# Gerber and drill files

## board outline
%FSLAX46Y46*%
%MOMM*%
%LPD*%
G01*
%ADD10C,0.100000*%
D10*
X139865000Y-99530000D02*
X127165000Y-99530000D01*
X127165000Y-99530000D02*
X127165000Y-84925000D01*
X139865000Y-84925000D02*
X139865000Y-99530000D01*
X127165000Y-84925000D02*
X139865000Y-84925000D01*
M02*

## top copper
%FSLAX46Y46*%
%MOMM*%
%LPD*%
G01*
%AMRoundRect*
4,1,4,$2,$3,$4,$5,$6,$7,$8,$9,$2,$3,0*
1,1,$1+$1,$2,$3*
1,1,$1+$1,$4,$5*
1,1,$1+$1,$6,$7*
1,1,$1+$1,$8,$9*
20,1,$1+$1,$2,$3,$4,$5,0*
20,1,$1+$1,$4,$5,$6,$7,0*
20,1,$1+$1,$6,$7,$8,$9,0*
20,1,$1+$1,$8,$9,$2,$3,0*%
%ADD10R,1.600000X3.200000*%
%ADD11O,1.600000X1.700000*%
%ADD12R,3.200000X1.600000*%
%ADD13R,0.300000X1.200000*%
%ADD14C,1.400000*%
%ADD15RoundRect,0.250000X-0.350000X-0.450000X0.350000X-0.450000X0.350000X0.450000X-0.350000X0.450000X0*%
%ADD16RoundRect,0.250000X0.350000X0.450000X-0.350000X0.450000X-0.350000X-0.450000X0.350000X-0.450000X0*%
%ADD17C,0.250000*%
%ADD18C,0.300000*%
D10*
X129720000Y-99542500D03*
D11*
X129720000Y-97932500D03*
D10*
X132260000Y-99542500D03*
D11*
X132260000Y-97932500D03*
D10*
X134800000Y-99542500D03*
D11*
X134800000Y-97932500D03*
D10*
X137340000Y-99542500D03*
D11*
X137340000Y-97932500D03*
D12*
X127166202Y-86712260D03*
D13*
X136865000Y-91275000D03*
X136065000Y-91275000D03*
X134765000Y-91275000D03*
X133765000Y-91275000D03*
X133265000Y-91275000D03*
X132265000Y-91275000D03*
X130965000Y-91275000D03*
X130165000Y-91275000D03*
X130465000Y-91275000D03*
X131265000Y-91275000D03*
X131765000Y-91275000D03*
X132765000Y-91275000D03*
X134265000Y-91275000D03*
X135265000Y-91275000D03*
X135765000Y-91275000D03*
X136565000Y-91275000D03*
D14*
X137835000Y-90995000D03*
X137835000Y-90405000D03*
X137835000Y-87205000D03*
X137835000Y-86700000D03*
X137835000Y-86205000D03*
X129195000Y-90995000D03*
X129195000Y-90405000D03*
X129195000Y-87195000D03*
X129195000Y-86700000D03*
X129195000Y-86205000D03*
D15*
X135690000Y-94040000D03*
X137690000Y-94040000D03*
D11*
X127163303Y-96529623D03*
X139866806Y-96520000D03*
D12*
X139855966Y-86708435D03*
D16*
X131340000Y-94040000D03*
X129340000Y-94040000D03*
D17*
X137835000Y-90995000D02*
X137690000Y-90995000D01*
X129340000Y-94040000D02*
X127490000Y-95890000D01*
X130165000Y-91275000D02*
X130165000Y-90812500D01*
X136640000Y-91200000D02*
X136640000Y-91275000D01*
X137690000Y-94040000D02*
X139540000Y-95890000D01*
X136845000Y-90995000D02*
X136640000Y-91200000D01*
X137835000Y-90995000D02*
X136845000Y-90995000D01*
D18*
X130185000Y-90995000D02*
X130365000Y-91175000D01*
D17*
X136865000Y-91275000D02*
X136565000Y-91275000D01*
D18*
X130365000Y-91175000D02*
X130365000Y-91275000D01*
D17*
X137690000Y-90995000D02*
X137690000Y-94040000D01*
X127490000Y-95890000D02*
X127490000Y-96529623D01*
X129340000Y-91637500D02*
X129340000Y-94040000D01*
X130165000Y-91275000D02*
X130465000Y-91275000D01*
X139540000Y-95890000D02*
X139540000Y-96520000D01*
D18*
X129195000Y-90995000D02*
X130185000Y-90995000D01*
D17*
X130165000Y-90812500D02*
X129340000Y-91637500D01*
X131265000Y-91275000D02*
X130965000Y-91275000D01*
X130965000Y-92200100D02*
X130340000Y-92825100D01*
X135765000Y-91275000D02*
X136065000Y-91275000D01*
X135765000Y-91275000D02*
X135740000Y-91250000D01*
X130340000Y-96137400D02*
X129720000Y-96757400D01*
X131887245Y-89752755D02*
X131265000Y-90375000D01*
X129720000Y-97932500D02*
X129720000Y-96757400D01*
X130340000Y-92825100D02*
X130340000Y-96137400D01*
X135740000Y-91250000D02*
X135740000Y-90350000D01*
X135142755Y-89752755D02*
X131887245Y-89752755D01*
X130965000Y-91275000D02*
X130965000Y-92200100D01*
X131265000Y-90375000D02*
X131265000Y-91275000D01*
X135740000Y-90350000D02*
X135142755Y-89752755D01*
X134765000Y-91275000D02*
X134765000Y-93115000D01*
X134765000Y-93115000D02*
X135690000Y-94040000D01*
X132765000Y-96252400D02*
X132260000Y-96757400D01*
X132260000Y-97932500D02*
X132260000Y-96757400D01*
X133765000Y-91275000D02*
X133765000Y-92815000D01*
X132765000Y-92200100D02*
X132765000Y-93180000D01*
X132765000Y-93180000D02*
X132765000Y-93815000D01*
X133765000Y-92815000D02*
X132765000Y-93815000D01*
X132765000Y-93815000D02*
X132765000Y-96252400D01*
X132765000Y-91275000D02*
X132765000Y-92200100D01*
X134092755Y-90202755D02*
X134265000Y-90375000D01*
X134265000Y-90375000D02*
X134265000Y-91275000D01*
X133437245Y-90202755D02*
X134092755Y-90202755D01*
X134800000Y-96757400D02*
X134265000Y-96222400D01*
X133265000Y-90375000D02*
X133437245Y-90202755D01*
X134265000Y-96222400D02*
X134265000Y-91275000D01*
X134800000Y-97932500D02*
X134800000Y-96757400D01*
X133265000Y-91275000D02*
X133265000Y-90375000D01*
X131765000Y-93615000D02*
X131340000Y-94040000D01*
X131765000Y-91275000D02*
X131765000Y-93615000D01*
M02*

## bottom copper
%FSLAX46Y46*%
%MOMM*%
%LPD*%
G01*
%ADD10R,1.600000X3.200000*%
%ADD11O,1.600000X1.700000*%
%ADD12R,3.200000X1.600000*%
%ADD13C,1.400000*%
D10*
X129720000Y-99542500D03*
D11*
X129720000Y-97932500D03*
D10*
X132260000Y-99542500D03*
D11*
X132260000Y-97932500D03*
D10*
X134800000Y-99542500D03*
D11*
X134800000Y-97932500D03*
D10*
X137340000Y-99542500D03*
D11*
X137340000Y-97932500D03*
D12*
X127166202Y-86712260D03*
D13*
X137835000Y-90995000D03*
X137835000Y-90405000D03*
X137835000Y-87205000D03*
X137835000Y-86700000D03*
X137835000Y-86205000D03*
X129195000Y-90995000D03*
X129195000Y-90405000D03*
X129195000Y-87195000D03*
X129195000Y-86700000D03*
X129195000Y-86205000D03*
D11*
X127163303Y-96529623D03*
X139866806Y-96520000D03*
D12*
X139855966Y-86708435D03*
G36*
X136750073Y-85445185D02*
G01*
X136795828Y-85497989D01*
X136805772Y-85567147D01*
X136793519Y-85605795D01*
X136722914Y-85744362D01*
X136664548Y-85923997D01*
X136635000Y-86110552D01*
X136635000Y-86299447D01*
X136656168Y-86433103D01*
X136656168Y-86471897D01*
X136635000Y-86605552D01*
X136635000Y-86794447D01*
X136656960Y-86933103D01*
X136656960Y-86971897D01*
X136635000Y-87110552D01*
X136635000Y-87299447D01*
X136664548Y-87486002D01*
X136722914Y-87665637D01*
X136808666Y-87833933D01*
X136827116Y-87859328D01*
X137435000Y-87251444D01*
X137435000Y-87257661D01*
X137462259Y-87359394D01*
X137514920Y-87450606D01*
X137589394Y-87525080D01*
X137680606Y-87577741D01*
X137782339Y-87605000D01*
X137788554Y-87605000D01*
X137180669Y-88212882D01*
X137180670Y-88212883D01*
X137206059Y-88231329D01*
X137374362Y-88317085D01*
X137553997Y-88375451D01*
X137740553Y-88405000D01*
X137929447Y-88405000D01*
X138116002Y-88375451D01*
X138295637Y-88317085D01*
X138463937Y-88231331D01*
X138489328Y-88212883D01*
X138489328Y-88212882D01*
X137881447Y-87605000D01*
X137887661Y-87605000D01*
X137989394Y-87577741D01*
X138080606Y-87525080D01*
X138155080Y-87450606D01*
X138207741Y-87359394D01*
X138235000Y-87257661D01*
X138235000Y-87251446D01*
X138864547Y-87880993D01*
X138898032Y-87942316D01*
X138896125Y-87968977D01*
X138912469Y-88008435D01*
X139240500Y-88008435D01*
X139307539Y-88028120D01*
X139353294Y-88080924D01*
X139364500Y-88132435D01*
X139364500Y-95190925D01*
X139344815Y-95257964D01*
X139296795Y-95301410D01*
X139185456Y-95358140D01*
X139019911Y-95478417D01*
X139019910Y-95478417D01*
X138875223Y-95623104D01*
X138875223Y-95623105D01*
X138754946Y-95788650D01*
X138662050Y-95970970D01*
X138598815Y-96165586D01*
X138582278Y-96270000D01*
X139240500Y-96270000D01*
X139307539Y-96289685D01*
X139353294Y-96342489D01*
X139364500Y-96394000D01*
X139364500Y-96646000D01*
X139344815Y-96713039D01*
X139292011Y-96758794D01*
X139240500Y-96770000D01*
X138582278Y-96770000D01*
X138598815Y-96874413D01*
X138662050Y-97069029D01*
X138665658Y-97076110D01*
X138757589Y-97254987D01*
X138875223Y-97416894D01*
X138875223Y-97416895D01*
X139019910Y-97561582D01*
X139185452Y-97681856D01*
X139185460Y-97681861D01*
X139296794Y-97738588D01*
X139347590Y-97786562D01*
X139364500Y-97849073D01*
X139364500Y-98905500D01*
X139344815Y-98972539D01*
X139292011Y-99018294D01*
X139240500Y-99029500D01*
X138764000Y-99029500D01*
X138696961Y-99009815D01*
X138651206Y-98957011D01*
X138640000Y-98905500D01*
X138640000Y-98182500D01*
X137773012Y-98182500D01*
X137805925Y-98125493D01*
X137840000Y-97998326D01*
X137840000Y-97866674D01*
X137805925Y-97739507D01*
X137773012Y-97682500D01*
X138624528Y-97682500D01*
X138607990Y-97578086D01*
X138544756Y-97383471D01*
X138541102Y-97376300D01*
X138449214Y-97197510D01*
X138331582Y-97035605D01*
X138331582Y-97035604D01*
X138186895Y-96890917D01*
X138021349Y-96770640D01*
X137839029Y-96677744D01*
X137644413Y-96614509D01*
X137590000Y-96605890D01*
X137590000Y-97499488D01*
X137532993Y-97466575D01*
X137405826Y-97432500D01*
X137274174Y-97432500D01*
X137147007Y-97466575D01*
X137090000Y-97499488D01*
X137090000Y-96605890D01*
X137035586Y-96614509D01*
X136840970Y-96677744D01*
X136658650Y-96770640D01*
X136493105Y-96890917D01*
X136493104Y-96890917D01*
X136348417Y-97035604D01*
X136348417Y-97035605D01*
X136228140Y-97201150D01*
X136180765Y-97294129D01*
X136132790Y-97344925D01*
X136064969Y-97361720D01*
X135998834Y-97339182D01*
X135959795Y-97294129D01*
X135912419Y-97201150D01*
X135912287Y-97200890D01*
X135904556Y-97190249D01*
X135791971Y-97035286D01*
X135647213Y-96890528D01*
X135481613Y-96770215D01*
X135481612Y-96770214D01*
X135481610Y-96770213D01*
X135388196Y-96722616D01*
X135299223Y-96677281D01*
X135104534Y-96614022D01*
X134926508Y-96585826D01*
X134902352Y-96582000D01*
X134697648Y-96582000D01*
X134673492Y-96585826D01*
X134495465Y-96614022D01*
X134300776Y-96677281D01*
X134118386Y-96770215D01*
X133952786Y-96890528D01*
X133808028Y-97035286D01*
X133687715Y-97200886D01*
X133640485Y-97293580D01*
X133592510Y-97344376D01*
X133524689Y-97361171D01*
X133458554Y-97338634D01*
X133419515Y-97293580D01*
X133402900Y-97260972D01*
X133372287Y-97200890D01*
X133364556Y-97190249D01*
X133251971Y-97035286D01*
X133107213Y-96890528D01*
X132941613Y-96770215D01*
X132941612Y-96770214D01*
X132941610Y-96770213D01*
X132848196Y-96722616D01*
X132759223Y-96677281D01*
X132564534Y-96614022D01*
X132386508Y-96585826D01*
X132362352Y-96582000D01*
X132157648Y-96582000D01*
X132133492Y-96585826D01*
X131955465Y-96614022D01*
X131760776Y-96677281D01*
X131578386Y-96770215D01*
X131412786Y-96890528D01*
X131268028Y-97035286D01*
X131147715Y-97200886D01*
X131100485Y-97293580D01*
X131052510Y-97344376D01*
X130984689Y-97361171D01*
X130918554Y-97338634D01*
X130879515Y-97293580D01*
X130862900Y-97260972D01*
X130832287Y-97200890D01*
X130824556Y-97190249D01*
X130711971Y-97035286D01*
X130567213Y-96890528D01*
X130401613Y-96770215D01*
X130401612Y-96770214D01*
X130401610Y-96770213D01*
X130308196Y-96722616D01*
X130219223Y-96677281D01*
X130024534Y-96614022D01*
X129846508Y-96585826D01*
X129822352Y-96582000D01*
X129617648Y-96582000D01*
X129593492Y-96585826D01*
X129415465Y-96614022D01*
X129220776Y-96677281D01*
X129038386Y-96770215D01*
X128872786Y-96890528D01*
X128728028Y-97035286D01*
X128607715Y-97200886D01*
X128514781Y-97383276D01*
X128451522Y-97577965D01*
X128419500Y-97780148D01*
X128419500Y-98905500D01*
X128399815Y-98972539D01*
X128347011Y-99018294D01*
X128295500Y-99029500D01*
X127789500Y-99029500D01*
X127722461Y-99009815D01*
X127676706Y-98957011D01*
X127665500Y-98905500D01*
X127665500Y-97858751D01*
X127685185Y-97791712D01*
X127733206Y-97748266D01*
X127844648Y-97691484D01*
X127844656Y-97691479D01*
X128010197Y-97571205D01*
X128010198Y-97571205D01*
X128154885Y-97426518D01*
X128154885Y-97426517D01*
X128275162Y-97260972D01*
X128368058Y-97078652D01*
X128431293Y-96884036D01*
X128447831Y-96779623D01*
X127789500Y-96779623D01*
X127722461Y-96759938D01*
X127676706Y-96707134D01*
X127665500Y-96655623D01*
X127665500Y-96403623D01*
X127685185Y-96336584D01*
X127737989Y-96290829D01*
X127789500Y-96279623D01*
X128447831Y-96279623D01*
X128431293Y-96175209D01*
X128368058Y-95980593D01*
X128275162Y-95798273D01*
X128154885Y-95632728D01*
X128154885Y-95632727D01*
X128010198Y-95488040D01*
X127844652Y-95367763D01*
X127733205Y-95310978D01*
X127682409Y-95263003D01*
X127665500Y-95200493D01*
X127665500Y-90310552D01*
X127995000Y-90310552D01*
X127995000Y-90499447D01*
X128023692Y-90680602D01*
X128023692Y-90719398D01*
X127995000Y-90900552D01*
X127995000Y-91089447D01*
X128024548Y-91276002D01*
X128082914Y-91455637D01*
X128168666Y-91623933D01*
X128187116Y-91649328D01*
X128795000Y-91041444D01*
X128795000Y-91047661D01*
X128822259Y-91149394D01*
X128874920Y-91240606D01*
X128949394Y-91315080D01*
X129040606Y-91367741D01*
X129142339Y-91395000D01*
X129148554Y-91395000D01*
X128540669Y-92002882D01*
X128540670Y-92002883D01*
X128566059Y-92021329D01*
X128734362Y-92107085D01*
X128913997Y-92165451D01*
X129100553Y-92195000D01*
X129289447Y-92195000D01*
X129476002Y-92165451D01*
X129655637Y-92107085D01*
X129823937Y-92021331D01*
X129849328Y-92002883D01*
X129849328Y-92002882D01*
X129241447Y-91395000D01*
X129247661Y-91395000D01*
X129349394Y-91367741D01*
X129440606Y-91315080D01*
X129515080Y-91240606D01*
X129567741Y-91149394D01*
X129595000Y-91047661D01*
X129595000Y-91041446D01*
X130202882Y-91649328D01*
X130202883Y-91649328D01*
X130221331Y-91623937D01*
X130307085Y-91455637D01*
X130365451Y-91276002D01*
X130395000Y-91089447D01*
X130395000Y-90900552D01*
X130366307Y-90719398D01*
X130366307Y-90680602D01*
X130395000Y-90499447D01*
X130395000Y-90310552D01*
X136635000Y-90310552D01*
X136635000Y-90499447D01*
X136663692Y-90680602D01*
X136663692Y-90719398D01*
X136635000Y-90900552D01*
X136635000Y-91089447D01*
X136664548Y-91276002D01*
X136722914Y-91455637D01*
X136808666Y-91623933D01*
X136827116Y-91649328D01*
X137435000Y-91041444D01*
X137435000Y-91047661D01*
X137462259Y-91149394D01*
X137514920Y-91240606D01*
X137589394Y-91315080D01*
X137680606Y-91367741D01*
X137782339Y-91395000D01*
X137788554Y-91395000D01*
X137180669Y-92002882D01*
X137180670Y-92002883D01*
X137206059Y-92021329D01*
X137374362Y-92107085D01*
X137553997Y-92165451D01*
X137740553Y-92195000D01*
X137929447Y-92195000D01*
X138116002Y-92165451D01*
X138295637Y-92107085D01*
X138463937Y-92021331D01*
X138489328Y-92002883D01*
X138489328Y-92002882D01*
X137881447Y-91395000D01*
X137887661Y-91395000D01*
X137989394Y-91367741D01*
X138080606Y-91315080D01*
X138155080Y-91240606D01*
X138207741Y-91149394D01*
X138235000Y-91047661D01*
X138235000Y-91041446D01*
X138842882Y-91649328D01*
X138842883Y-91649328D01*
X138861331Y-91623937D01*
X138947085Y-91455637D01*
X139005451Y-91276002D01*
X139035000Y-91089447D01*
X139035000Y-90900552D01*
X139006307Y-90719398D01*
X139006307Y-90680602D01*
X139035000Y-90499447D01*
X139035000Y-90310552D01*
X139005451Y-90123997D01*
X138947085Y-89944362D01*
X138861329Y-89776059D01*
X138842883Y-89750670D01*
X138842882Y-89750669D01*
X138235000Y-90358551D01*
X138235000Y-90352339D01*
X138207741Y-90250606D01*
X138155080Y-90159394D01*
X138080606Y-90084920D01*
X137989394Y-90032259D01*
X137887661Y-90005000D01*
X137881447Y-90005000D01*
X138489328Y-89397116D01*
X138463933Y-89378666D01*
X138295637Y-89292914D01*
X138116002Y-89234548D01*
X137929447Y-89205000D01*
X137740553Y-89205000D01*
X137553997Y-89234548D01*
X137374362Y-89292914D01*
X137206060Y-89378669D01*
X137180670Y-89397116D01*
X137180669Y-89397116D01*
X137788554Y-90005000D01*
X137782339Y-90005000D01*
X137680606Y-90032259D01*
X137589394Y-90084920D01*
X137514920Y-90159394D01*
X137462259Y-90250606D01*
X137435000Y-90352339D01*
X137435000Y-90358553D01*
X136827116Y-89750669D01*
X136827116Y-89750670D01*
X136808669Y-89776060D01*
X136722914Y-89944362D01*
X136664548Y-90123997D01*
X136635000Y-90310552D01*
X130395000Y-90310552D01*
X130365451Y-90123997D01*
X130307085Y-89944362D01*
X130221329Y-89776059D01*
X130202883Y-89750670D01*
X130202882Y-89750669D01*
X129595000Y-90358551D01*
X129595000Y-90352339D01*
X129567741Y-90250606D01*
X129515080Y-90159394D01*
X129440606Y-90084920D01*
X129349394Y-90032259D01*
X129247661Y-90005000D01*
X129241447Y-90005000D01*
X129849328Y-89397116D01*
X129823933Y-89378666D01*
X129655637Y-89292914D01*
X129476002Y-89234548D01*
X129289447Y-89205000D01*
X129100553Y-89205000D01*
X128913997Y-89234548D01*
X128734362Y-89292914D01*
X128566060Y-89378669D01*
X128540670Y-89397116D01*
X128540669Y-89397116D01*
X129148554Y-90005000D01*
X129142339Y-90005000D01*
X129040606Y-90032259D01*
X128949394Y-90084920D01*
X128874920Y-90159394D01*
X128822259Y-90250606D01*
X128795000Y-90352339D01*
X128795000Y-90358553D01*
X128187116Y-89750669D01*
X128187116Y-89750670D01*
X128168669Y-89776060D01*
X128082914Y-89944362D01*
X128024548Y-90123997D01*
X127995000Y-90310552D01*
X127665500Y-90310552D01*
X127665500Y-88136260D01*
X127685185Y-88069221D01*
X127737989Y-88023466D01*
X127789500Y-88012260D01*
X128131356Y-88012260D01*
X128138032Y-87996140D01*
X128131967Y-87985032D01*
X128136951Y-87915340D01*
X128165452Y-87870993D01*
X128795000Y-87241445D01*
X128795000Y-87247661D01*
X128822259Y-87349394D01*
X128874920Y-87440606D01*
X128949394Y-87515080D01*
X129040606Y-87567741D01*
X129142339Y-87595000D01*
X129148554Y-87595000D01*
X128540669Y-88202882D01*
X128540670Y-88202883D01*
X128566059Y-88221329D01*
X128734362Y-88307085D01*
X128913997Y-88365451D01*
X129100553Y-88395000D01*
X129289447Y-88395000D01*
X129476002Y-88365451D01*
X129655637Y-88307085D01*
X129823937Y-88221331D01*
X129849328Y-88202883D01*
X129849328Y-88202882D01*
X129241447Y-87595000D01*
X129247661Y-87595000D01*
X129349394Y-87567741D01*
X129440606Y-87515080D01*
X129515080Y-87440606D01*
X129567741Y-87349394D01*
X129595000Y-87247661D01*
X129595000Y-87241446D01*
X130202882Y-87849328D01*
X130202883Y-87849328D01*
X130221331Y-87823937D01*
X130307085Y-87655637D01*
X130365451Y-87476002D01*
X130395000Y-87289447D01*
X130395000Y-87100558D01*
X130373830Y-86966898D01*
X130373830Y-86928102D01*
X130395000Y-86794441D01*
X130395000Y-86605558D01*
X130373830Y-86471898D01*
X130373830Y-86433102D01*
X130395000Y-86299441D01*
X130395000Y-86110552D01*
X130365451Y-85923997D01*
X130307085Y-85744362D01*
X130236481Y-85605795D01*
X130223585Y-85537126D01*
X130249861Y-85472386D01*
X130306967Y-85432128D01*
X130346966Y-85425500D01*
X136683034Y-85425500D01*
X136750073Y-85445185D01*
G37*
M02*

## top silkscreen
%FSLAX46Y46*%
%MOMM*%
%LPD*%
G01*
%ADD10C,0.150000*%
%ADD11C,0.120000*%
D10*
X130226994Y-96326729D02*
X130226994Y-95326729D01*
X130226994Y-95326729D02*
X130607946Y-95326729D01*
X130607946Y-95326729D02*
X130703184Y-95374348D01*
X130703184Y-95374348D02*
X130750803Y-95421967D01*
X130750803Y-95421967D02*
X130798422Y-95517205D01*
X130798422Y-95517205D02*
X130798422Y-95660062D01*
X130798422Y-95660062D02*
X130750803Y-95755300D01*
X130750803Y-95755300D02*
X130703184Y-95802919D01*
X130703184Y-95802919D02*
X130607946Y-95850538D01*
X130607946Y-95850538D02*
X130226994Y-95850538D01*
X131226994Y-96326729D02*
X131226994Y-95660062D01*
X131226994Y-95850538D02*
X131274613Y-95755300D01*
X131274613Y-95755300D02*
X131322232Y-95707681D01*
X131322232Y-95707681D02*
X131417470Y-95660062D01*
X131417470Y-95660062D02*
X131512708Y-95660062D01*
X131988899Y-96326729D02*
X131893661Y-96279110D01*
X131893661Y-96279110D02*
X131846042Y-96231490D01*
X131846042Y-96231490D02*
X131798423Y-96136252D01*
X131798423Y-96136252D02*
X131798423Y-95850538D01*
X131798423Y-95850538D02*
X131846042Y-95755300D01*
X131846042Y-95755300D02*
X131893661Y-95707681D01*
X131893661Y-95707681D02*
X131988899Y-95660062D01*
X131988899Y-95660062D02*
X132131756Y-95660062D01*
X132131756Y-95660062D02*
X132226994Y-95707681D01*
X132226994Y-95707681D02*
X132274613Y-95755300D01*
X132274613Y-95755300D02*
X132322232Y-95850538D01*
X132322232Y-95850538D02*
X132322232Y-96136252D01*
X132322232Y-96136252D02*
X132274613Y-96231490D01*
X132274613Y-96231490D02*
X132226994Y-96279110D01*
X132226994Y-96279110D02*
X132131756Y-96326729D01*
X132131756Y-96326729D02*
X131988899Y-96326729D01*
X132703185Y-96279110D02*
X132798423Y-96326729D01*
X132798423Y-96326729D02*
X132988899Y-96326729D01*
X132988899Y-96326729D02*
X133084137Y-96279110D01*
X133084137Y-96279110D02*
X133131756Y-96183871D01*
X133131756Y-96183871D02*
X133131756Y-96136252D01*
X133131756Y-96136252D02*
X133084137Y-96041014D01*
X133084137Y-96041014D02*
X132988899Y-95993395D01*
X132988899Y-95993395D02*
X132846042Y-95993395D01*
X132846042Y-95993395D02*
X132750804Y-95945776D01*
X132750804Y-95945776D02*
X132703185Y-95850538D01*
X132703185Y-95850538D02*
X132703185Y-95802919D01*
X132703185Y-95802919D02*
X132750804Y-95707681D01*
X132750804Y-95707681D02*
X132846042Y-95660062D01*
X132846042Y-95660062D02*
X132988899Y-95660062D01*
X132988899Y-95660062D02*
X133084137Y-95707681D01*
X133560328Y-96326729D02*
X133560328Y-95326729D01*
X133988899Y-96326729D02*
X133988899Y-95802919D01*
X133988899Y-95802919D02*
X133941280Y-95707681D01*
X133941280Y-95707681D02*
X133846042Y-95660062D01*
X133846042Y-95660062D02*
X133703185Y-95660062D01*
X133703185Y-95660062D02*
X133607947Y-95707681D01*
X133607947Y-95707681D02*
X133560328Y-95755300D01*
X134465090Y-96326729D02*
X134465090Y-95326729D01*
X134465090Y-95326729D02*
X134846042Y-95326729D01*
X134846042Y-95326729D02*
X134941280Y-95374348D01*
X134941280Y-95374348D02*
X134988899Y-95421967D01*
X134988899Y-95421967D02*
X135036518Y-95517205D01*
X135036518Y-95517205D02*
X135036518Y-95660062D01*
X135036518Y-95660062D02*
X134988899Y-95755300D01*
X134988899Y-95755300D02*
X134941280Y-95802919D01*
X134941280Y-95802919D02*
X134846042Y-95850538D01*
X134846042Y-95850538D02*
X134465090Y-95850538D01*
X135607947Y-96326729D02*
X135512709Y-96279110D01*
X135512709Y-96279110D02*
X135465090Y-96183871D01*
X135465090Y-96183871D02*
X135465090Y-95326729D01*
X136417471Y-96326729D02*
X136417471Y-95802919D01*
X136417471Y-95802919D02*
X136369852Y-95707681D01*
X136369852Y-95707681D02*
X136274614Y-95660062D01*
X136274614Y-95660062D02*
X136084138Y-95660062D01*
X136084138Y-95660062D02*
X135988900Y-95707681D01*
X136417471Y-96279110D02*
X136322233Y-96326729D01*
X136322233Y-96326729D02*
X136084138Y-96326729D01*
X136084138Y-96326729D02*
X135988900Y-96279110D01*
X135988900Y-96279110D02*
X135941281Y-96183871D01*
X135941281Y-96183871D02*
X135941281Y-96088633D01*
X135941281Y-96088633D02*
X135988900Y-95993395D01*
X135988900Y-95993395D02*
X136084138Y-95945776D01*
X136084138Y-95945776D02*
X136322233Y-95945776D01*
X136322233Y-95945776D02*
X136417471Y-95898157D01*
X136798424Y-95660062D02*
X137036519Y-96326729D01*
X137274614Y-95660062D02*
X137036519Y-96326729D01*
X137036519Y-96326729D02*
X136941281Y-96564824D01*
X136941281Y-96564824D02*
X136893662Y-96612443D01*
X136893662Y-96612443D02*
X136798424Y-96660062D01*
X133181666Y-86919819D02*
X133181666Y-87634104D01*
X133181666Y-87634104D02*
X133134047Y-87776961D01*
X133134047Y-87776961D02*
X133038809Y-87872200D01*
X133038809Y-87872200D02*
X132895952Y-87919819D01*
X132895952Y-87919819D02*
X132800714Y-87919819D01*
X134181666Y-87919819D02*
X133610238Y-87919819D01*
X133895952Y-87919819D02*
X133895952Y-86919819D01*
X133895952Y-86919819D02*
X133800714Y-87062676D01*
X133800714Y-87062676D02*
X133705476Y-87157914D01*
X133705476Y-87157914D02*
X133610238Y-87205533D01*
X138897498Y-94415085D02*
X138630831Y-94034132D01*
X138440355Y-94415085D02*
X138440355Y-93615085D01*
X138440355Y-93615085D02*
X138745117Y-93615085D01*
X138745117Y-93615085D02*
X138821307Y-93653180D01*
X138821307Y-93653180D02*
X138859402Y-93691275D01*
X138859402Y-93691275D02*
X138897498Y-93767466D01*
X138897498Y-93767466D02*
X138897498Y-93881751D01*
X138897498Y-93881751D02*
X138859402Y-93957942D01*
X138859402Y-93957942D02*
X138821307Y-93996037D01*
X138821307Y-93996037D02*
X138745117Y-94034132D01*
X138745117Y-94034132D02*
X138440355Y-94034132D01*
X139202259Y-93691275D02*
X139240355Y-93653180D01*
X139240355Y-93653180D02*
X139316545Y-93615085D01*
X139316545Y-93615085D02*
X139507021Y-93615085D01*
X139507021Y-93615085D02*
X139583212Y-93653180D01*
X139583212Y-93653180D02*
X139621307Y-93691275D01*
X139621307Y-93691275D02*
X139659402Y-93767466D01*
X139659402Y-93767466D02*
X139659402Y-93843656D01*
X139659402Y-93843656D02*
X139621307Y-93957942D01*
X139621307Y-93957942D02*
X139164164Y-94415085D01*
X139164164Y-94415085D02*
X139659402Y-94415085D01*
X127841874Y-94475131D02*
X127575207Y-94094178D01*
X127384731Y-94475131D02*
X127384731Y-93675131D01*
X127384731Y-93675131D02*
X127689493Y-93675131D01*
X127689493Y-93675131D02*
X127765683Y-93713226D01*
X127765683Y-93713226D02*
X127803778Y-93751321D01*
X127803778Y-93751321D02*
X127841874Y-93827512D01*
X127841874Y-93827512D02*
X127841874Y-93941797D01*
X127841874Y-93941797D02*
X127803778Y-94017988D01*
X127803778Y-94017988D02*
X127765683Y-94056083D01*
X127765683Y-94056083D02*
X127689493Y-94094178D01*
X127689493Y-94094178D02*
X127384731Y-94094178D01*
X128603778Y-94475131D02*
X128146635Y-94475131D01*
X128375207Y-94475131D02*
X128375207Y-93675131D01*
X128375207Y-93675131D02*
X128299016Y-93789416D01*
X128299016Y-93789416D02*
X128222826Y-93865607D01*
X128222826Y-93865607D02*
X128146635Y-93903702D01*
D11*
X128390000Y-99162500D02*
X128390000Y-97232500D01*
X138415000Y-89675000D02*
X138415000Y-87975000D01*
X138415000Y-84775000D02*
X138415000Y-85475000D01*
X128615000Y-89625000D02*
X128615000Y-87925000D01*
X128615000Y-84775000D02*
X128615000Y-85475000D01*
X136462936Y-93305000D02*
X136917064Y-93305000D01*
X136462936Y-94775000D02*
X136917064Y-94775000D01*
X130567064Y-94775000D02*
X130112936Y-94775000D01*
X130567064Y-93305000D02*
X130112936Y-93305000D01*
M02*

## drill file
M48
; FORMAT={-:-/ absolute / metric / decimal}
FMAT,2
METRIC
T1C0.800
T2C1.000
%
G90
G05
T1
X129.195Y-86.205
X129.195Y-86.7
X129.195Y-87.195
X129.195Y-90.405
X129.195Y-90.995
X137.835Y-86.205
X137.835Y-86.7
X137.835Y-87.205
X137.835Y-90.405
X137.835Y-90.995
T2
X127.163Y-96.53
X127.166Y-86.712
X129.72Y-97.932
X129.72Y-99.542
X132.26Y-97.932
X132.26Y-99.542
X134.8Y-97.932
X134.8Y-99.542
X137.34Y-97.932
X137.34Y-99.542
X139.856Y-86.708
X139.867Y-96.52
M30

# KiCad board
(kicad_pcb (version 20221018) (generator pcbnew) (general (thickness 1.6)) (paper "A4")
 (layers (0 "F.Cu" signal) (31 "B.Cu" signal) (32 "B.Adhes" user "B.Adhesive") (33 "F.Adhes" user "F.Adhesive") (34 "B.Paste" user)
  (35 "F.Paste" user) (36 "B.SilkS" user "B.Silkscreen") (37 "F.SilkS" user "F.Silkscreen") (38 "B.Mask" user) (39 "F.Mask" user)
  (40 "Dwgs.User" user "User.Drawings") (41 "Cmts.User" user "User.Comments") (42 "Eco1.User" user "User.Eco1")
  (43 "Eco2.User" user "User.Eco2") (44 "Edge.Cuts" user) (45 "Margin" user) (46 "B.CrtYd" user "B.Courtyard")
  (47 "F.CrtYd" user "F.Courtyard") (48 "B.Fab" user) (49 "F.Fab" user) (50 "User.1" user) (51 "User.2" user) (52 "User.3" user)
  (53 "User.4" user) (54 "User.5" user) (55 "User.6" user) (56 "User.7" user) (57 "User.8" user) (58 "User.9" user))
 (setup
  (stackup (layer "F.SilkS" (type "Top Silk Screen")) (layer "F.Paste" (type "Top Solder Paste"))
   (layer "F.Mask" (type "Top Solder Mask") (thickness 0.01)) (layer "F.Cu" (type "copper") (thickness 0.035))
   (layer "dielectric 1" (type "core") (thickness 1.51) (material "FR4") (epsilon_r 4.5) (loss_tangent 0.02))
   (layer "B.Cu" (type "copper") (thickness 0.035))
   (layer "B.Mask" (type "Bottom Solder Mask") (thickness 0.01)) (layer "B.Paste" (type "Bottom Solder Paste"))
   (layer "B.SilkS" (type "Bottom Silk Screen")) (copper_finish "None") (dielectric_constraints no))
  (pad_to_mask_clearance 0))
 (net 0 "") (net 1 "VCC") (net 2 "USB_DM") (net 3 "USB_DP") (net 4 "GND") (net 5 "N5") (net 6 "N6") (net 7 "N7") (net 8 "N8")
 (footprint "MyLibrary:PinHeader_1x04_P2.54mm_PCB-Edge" (layer "F.Cu") (at 129.72 97.9325 90)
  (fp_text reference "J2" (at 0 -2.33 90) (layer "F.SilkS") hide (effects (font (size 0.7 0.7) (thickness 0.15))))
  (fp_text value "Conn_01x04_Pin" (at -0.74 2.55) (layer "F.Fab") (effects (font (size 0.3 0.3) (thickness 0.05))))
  (fp_line (start -1.23 -1.33) (end 0.7 -1.33) (stroke (width 0.12) (type solid)) (layer "F.SilkS"))
  (pad "1" thru_hole rect (at -1.61 0 90) (size 3.2 1.6) (drill 1) (layers "*.Cu" "*.Mask") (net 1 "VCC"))
  (pad "1" thru_hole oval (at 0 0 90) (size 1.7 1.6) (drill 1) (layers "*.Cu" "*.Mask") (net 1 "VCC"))
  (pad "2" thru_hole rect (at -1.61 2.54 90) (size 3.2 1.6) (drill 1) (layers "*.Cu" "*.Mask") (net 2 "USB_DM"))
  (pad "2" thru_hole oval (at 0 2.54 90) (size 1.7 1.6) (drill 1) (layers "*.Cu" "*.Mask") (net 2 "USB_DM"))
  (pad "3" thru_hole rect (at -1.61 5.08 90) (size 3.2 1.6) (drill 1) (layers "*.Cu" "*.Mask") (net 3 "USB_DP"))
  (pad "3" thru_hole oval (at 0 5.08 90) (size 1.7 1.6) (drill 1) (layers "*.Cu" "*.Mask") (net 3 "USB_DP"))
  (pad "4" thru_hole rect (at -1.61 7.62 90) (size 3.2 1.6) (drill 1) (layers "*.Cu" "*.Mask") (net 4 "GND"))
  (pad "4" thru_hole oval (at 0 7.62 90) (size 1.7 1.6) (drill 1) (layers "*.Cu" "*.Mask") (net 4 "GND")))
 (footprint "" (layer "F.Cu") (at 127.166202 86.71226 -90)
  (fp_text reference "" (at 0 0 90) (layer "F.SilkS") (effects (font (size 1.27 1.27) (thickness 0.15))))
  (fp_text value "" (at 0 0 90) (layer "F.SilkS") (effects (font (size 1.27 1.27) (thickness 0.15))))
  (pad "4" thru_hole rect (at 0 0) (size 3.2 1.6) (drill 1) (layers "*.Cu" "*.Mask") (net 4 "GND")))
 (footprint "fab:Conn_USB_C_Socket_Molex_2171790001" (layer "F.Cu") (at 133.515 91.275 180)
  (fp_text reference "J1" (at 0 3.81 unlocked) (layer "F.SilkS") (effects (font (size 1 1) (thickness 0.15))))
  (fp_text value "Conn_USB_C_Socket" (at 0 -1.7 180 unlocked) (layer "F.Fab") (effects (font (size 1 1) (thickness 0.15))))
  (fp_line (start -4.9 1.6) (end -4.9 3.3) (stroke (width 0.12) (type solid)) (layer "F.SilkS"))
  (fp_line (start -4.9 6.5) (end -4.9 5.8) (stroke (width 0.12) (type solid)) (layer "F.SilkS"))
  (fp_line (start 4.9 1.65) (end 4.9 3.35) (stroke (width 0.12) (type solid)) (layer "F.SilkS"))
  (fp_line (start 4.9 6.5) (end 4.9 5.8) (stroke (width 0.12) (type solid)) (layer "F.SilkS"))
  (pad "A1" smd rect (at -3.35 0 180) (size 0.3 1.2) (layers "F.Cu" "F.Paste" "F.Mask") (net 4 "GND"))
  (pad "A4" smd rect (at -2.55 0 180) (size 0.3 1.2) (layers "F.Cu" "F.Paste" "F.Mask") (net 1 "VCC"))
  (pad "A5" smd rect (at -1.25 0 180) (size 0.3 1.2) (layers "F.Cu" "F.Paste" "F.Mask") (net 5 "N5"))
  (pad "A6" smd rect (at -0.25 0 180) (size 0.3 1.2) (layers "F.Cu" "F.Paste" "F.Mask") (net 2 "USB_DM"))
  (pad "A7" smd rect (at 0.25 0 180) (size 0.3 1.2) (layers "F.Cu" "F.Paste" "F.Mask") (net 3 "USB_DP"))
  (pad "A8" smd rect (at 1.25 0 180) (size 0.3 1.2) (layers "F.Cu" "F.Paste" "F.Mask") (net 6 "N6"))
  (pad "A9" smd rect (at 2.55 0 180) (size 0.3 1.2) (layers "F.Cu" "F.Paste" "F.Mask") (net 1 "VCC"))
  (pad "A12" smd rect (at 3.35 0 180) (size 0.3 1.2) (layers "F.Cu" "F.Paste" "F.Mask") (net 4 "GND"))
  (pad "B1" smd rect (at 3.05 0 180) (size 0.3 1.2) (layers "F.Cu" "F.Paste" "F.Mask") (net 4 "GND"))
  (pad "B4" smd rect (at 2.25 0 180) (size 0.3 1.2) (layers "F.Cu" "F.Paste" "F.Mask") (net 1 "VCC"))
  (pad "B5" smd rect (at 1.75 0 180) (size 0.3 1.2) (layers "F.Cu" "F.Paste" "F.Mask") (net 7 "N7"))
  (pad "B6" smd rect (at 0.75 0 180) (size 0.3 1.2) (layers "F.Cu" "F.Paste" "F.Mask") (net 2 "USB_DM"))
  (pad "B7" smd rect (at -0.75 0 180) (size 0.3 1.2) (layers "F.Cu" "F.Paste" "F.Mask") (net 3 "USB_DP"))
  (pad "B8" smd rect (at -1.75 0 180) (size 0.3 1.2) (layers "F.Cu" "F.Paste" "F.Mask") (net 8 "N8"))
  (pad "B9" smd rect (at -2.25 0 180) (size 0.3 1.2) (layers "F.Cu" "F.Paste" "F.Mask") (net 1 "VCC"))
  (pad "B12" smd rect (at -3.05 0 180) (size 0.3 1.2) (layers "F.Cu" "F.Paste" "F.Mask") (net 4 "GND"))
  (pad "S1" thru_hole circle (at -4.32 0.28 180) (size 1.4 1.4) (drill 0.8) (layers "*.Cu" "*.Mask") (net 4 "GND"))
  (pad "S1" thru_hole circle (at -4.32 0.87 180) (size 1.4 1.4) (drill 0.8) (layers "*.Cu" "*.Mask") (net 4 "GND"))
  (pad "S1" thru_hole circle (at -4.32 4.07 180) (size 1.4 1.4) (drill 0.8) (layers "*.Cu" "*.Mask") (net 4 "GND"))
  (pad "S1" thru_hole circle (at -4.32 4.575 180) (size 1.4 1.4) (drill 0.8) (layers "*.Cu" "*.Mask") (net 4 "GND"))
  (pad "S1" thru_hole circle (at -4.32 5.07 180) (size 1.4 1.4) (drill 0.8) (layers "*.Cu" "*.Mask") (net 4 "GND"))
  (pad "S1" thru_hole circle (at 4.32 0.28 180) (size 1.4 1.4) (drill 0.8) (layers "*.Cu" "*.Mask") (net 4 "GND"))
  (pad "S1" thru_hole circle (at 4.32 0.87 180) (size 1.4 1.4) (drill 0.8) (layers "*.Cu" "*.Mask") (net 4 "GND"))
  (pad "S1" thru_hole circle (at 4.32 4.08 180) (size 1.4 1.4) (drill 0.8) (layers "*.Cu" "*.Mask") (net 4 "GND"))
  (pad "S1" thru_hole circle (at 4.32 4.575 180) (size 1.4 1.4) (drill 0.8) (layers "*.Cu" "*.Mask") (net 4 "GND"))
  (pad "S1" thru_hole circle (at 4.32 5.07 180) (size 1.4 1.4) (drill 0.8) (layers "*.Cu" "*.Mask") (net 4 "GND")))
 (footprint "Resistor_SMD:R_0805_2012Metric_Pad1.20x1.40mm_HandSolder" (layer "F.Cu") (at 136.69 94.04)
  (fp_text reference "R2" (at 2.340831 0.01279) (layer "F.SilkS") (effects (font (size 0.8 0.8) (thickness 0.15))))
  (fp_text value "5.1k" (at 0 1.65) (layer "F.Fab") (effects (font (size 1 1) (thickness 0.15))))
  (fp_line (start -0.227064 -0.735) (end 0.227064 -0.735) (stroke (width 0.12) (type solid)) (layer "F.SilkS"))
  (fp_line (start -0.227064 0.735) (end 0.227064 0.735) (stroke (width 0.12) (type solid)) (layer "F.SilkS"))
  (pad "1" smd roundrect (at -1 0) (size 1.2 1.4) (layers "F.Cu" "F.Paste" "F.Mask") (roundrect_rratio 0.2083333333) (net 5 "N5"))
  (pad "2" smd roundrect (at 1 0) (size 1.2 1.4) (layers "F.Cu" "F.Paste" "F.Mask") (roundrect_rratio 0.2083333333) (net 4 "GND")))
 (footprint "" (layer "F.Cu") (at 127.163303 96.529623)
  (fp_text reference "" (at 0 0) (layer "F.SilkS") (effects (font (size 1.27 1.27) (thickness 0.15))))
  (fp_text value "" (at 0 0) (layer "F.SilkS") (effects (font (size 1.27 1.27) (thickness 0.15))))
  (pad "4" thru_hole oval (at 0 0 90) (size 1.7 1.6) (drill 1) (layers "*.Cu" "*.Mask") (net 4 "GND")))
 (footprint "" (layer "F.Cu") (at 139.866806 96.52)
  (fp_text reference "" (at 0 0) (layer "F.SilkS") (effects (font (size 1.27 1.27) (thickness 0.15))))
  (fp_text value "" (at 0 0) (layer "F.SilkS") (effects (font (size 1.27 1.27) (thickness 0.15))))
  (pad "4" thru_hole oval (at 0 0 90) (size 1.7 1.6) (drill 1) (layers "*.Cu" "*.Mask") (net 4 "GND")))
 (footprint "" (layer "F.Cu") (at 139.855966 86.708435 180)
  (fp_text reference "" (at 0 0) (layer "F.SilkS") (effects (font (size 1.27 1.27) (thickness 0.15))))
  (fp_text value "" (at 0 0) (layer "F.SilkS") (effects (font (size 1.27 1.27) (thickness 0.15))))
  (pad "4" thru_hole rect (at 0 0 180) (size 3.2 1.6) (drill 1) (layers "*.Cu" "*.Mask") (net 4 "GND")))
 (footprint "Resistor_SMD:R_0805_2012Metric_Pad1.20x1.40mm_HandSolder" (layer "F.Cu") (at 130.34 94.04 180)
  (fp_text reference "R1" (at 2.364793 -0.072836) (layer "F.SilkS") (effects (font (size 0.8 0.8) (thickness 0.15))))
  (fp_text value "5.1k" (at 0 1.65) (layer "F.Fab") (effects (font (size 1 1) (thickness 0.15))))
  (fp_line (start -0.227064 -0.735) (end 0.227064 -0.735) (stroke (width 0.12) (type solid)) (layer "F.SilkS"))
  (fp_line (start -0.227064 0.735) (end 0.227064 0.735) (stroke (width 0.12) (type solid)) (layer "F.SilkS"))
  (pad "1" smd roundrect (at -1 0 180) (size 1.2 1.4) (layers "F.Cu" "F.Paste" "F.Mask") (roundrect_rratio 0.2083333333) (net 7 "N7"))
  (pad "2" smd roundrect (at 1 0 180) (size 1.2 1.4) (layers "F.Cu" "F.Paste" "F.Mask") (roundrect_rratio 0.2083333333) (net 4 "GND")))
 (gr_line (start 139.865 99.53) (end 127.165 99.53) (stroke (width 0.1) (type default)) (layer "Edge.Cuts"))
 (gr_line (start 127.165 99.53) (end 127.165 84.925) (stroke (width 0.1) (type default)) (layer "Edge.Cuts"))
 (gr_line (start 139.865 84.925) (end 139.865 99.53) (stroke (width 0.1) (type default)) (layer "Edge.Cuts"))
 (gr_line (start 127.165 84.925) (end 139.865 84.925) (stroke (width 0.1) (type default)) (layer "Edge.Cuts"))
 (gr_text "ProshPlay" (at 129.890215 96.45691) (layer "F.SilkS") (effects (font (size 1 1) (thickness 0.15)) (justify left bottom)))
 (segment (start 137.835 90.995) (end 137.69 90.995) (width 0.25) (layer "F.Cu") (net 4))
 (segment (start 129.34 94.04) (end 127.49 95.89) (width 0.25) (layer "F.Cu") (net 4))
 (segment (start 130.165 91.275) (end 130.165 90.8125) (width 0.25) (layer "F.Cu") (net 4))
 (segment (start 136.64 91.2) (end 136.64 91.275) (width 0.25) (layer "F.Cu") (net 4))
 (segment (start 137.69 94.04) (end 139.54 95.89) (width 0.25) (layer "F.Cu") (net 4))
 (segment (start 136.845 90.995) (end 136.64 91.2) (width 0.25) (layer "F.Cu") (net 4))
 (segment (start 137.835 90.995) (end 136.845 90.995) (width 0.25) (layer "F.Cu") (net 4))
 (segment (start 130.185 90.995) (end 130.365 91.175) (width 0.3) (layer "F.Cu") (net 4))
 (segment (start 136.865 91.275) (end 136.565 91.275) (width 0.25) (layer "F.Cu") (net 4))
 (segment (start 130.365 91.175) (end 130.365 91.275) (width 0.3) (layer "F.Cu") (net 4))
 (segment (start 137.69 90.995) (end 137.69 94.04) (width 0.25) (layer "F.Cu") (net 4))
 (segment (start 127.49 95.89) (end 127.49 96.529623) (width 0.25) (layer "F.Cu") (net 4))
 (segment (start 129.34 91.6375) (end 129.34 94.04) (width 0.25) (layer "F.Cu") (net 4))
 (segment (start 130.165 91.275) (end 130.465 91.275) (width 0.25) (layer "F.Cu") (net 4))
 (segment (start 139.54 95.89) (end 139.54 96.52) (width 0.25) (layer "F.Cu") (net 4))
 (segment (start 129.195 90.995) (end 130.185 90.995) (width 0.3) (layer "F.Cu") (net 4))
 (segment (start 130.165 90.8125) (end 129.34 91.6375) (width 0.25) (layer "F.Cu") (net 4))
 (segment (start 131.265 91.275) (end 130.965 91.275) (width 0.25) (layer "F.Cu") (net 1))
 (segment (start 130.965 92.2001) (end 130.34 92.8251) (width 0.25) (layer "F.Cu") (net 1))
 (segment (start 135.765 91.275) (end 136.065 91.275) (width 0.25) (layer "F.Cu") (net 1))
 (segment (start 135.765 91.275) (end 135.74 91.25) (width 0.25) (layer "F.Cu") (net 1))
 (segment (start 130.34 96.1374) (end 129.72 96.7574) (width 0.25) (layer "F.Cu") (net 1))
 (segment (start 131.887245 89.752755) (end 131.265 90.375) (width 0.25) (layer "F.Cu") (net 1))
 (segment (start 129.72 97.9325) (end 129.72 96.7574) (width 0.25) (layer "F.Cu") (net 1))
 (segment (start 130.34 92.8251) (end 130.34 96.1374) (width 0.25) (layer "F.Cu") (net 1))
 (segment (start 135.74 91.25) (end 135.74 90.35) (width 0.25) (layer "F.Cu") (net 1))
 (segment (start 135.142755 89.752755) (end 131.887245 89.752755) (width 0.25) (layer "F.Cu") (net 1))
 (segment (start 130.965 91.275) (end 130.965 92.2001) (width 0.25) (layer "F.Cu") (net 1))
 (segment (start 131.265 90.375) (end 131.265 91.275) (width 0.25) (layer "F.Cu") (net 1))
 (segment (start 135.74 90.35) (end 135.142755 89.752755) (width 0.25) (layer "F.Cu") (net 1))
 (segment (start 134.765 91.275) (end 134.765 93.115) (width 0.25) (layer "F.Cu") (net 5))
 (segment (start 134.765 93.115) (end 135.69 94.04) (width 0.25) (layer "F.Cu") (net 5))
 (segment (start 132.765 96.2524) (end 132.26 96.7574) (width 0.25) (layer "F.Cu") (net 2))
 (segment (start 132.26 97.9325) (end 132.26 96.7574) (width 0.25) (layer "F.Cu") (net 2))
 (segment (start 133.765 91.275) (end 133.765 92.815) (width 0.25) (layer "F.Cu") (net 2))
 (segment (start 132.765 92.2001) (end 132.765 93.18) (width 0.25) (layer "F.Cu") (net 2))
 (segment (start 132.765 93.18) (end 132.765 93.815) (width 0.25) (layer "F.Cu") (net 2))
 (segment (start 133.765 92.815) (end 132.765 93.815) (width 0.25) (layer "F.Cu") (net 2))
 (segment (start 132.765 93.815) (end 132.765 96.2524) (width 0.25) (layer "F.Cu") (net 2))
 (segment (start 132.765 91.275) (end 132.765 92.2001) (width 0.25) (layer "F.Cu") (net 2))
 (segment (start 134.092755 90.202755) (end 134.265 90.375) (width 0.25) (layer "F.Cu") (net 3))
 (segment (start 134.265 90.375) (end 134.265 91.275) (width 0.25) (layer "F.Cu") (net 3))
 (segment (start 133.437245 90.202755) (end 134.092755 90.202755) (width 0.25) (layer "F.Cu") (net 3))
 (segment (start 134.8 96.7574) (end 134.265 96.2224) (width 0.25) (layer "F.Cu") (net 3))
 (segment (start 133.265 90.375) (end 133.437245 90.202755) (width 0.25) (layer "F.Cu") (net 3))
 (segment (start 134.265 96.2224) (end 134.265 91.275) (width 0.25) (layer "F.Cu") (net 3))
 (segment (start 134.8 97.9325) (end 134.8 96.7574) (width 0.25) (layer "F.Cu") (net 3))
 (segment (start 133.265 91.275) (end 133.265 90.375) (width 0.25) (layer "F.Cu") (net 3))
 (segment (start 131.765 93.615) (end 131.34 94.04) (width 0.25) (layer "F.Cu") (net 7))
 (segment (start 131.765 91.275) (end 131.765 93.615) (width 0.25) (layer "F.Cu") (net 7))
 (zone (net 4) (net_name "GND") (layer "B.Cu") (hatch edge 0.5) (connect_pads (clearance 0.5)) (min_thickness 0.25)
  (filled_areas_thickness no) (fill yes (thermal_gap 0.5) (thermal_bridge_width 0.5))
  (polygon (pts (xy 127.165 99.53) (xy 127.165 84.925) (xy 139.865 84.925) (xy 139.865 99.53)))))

